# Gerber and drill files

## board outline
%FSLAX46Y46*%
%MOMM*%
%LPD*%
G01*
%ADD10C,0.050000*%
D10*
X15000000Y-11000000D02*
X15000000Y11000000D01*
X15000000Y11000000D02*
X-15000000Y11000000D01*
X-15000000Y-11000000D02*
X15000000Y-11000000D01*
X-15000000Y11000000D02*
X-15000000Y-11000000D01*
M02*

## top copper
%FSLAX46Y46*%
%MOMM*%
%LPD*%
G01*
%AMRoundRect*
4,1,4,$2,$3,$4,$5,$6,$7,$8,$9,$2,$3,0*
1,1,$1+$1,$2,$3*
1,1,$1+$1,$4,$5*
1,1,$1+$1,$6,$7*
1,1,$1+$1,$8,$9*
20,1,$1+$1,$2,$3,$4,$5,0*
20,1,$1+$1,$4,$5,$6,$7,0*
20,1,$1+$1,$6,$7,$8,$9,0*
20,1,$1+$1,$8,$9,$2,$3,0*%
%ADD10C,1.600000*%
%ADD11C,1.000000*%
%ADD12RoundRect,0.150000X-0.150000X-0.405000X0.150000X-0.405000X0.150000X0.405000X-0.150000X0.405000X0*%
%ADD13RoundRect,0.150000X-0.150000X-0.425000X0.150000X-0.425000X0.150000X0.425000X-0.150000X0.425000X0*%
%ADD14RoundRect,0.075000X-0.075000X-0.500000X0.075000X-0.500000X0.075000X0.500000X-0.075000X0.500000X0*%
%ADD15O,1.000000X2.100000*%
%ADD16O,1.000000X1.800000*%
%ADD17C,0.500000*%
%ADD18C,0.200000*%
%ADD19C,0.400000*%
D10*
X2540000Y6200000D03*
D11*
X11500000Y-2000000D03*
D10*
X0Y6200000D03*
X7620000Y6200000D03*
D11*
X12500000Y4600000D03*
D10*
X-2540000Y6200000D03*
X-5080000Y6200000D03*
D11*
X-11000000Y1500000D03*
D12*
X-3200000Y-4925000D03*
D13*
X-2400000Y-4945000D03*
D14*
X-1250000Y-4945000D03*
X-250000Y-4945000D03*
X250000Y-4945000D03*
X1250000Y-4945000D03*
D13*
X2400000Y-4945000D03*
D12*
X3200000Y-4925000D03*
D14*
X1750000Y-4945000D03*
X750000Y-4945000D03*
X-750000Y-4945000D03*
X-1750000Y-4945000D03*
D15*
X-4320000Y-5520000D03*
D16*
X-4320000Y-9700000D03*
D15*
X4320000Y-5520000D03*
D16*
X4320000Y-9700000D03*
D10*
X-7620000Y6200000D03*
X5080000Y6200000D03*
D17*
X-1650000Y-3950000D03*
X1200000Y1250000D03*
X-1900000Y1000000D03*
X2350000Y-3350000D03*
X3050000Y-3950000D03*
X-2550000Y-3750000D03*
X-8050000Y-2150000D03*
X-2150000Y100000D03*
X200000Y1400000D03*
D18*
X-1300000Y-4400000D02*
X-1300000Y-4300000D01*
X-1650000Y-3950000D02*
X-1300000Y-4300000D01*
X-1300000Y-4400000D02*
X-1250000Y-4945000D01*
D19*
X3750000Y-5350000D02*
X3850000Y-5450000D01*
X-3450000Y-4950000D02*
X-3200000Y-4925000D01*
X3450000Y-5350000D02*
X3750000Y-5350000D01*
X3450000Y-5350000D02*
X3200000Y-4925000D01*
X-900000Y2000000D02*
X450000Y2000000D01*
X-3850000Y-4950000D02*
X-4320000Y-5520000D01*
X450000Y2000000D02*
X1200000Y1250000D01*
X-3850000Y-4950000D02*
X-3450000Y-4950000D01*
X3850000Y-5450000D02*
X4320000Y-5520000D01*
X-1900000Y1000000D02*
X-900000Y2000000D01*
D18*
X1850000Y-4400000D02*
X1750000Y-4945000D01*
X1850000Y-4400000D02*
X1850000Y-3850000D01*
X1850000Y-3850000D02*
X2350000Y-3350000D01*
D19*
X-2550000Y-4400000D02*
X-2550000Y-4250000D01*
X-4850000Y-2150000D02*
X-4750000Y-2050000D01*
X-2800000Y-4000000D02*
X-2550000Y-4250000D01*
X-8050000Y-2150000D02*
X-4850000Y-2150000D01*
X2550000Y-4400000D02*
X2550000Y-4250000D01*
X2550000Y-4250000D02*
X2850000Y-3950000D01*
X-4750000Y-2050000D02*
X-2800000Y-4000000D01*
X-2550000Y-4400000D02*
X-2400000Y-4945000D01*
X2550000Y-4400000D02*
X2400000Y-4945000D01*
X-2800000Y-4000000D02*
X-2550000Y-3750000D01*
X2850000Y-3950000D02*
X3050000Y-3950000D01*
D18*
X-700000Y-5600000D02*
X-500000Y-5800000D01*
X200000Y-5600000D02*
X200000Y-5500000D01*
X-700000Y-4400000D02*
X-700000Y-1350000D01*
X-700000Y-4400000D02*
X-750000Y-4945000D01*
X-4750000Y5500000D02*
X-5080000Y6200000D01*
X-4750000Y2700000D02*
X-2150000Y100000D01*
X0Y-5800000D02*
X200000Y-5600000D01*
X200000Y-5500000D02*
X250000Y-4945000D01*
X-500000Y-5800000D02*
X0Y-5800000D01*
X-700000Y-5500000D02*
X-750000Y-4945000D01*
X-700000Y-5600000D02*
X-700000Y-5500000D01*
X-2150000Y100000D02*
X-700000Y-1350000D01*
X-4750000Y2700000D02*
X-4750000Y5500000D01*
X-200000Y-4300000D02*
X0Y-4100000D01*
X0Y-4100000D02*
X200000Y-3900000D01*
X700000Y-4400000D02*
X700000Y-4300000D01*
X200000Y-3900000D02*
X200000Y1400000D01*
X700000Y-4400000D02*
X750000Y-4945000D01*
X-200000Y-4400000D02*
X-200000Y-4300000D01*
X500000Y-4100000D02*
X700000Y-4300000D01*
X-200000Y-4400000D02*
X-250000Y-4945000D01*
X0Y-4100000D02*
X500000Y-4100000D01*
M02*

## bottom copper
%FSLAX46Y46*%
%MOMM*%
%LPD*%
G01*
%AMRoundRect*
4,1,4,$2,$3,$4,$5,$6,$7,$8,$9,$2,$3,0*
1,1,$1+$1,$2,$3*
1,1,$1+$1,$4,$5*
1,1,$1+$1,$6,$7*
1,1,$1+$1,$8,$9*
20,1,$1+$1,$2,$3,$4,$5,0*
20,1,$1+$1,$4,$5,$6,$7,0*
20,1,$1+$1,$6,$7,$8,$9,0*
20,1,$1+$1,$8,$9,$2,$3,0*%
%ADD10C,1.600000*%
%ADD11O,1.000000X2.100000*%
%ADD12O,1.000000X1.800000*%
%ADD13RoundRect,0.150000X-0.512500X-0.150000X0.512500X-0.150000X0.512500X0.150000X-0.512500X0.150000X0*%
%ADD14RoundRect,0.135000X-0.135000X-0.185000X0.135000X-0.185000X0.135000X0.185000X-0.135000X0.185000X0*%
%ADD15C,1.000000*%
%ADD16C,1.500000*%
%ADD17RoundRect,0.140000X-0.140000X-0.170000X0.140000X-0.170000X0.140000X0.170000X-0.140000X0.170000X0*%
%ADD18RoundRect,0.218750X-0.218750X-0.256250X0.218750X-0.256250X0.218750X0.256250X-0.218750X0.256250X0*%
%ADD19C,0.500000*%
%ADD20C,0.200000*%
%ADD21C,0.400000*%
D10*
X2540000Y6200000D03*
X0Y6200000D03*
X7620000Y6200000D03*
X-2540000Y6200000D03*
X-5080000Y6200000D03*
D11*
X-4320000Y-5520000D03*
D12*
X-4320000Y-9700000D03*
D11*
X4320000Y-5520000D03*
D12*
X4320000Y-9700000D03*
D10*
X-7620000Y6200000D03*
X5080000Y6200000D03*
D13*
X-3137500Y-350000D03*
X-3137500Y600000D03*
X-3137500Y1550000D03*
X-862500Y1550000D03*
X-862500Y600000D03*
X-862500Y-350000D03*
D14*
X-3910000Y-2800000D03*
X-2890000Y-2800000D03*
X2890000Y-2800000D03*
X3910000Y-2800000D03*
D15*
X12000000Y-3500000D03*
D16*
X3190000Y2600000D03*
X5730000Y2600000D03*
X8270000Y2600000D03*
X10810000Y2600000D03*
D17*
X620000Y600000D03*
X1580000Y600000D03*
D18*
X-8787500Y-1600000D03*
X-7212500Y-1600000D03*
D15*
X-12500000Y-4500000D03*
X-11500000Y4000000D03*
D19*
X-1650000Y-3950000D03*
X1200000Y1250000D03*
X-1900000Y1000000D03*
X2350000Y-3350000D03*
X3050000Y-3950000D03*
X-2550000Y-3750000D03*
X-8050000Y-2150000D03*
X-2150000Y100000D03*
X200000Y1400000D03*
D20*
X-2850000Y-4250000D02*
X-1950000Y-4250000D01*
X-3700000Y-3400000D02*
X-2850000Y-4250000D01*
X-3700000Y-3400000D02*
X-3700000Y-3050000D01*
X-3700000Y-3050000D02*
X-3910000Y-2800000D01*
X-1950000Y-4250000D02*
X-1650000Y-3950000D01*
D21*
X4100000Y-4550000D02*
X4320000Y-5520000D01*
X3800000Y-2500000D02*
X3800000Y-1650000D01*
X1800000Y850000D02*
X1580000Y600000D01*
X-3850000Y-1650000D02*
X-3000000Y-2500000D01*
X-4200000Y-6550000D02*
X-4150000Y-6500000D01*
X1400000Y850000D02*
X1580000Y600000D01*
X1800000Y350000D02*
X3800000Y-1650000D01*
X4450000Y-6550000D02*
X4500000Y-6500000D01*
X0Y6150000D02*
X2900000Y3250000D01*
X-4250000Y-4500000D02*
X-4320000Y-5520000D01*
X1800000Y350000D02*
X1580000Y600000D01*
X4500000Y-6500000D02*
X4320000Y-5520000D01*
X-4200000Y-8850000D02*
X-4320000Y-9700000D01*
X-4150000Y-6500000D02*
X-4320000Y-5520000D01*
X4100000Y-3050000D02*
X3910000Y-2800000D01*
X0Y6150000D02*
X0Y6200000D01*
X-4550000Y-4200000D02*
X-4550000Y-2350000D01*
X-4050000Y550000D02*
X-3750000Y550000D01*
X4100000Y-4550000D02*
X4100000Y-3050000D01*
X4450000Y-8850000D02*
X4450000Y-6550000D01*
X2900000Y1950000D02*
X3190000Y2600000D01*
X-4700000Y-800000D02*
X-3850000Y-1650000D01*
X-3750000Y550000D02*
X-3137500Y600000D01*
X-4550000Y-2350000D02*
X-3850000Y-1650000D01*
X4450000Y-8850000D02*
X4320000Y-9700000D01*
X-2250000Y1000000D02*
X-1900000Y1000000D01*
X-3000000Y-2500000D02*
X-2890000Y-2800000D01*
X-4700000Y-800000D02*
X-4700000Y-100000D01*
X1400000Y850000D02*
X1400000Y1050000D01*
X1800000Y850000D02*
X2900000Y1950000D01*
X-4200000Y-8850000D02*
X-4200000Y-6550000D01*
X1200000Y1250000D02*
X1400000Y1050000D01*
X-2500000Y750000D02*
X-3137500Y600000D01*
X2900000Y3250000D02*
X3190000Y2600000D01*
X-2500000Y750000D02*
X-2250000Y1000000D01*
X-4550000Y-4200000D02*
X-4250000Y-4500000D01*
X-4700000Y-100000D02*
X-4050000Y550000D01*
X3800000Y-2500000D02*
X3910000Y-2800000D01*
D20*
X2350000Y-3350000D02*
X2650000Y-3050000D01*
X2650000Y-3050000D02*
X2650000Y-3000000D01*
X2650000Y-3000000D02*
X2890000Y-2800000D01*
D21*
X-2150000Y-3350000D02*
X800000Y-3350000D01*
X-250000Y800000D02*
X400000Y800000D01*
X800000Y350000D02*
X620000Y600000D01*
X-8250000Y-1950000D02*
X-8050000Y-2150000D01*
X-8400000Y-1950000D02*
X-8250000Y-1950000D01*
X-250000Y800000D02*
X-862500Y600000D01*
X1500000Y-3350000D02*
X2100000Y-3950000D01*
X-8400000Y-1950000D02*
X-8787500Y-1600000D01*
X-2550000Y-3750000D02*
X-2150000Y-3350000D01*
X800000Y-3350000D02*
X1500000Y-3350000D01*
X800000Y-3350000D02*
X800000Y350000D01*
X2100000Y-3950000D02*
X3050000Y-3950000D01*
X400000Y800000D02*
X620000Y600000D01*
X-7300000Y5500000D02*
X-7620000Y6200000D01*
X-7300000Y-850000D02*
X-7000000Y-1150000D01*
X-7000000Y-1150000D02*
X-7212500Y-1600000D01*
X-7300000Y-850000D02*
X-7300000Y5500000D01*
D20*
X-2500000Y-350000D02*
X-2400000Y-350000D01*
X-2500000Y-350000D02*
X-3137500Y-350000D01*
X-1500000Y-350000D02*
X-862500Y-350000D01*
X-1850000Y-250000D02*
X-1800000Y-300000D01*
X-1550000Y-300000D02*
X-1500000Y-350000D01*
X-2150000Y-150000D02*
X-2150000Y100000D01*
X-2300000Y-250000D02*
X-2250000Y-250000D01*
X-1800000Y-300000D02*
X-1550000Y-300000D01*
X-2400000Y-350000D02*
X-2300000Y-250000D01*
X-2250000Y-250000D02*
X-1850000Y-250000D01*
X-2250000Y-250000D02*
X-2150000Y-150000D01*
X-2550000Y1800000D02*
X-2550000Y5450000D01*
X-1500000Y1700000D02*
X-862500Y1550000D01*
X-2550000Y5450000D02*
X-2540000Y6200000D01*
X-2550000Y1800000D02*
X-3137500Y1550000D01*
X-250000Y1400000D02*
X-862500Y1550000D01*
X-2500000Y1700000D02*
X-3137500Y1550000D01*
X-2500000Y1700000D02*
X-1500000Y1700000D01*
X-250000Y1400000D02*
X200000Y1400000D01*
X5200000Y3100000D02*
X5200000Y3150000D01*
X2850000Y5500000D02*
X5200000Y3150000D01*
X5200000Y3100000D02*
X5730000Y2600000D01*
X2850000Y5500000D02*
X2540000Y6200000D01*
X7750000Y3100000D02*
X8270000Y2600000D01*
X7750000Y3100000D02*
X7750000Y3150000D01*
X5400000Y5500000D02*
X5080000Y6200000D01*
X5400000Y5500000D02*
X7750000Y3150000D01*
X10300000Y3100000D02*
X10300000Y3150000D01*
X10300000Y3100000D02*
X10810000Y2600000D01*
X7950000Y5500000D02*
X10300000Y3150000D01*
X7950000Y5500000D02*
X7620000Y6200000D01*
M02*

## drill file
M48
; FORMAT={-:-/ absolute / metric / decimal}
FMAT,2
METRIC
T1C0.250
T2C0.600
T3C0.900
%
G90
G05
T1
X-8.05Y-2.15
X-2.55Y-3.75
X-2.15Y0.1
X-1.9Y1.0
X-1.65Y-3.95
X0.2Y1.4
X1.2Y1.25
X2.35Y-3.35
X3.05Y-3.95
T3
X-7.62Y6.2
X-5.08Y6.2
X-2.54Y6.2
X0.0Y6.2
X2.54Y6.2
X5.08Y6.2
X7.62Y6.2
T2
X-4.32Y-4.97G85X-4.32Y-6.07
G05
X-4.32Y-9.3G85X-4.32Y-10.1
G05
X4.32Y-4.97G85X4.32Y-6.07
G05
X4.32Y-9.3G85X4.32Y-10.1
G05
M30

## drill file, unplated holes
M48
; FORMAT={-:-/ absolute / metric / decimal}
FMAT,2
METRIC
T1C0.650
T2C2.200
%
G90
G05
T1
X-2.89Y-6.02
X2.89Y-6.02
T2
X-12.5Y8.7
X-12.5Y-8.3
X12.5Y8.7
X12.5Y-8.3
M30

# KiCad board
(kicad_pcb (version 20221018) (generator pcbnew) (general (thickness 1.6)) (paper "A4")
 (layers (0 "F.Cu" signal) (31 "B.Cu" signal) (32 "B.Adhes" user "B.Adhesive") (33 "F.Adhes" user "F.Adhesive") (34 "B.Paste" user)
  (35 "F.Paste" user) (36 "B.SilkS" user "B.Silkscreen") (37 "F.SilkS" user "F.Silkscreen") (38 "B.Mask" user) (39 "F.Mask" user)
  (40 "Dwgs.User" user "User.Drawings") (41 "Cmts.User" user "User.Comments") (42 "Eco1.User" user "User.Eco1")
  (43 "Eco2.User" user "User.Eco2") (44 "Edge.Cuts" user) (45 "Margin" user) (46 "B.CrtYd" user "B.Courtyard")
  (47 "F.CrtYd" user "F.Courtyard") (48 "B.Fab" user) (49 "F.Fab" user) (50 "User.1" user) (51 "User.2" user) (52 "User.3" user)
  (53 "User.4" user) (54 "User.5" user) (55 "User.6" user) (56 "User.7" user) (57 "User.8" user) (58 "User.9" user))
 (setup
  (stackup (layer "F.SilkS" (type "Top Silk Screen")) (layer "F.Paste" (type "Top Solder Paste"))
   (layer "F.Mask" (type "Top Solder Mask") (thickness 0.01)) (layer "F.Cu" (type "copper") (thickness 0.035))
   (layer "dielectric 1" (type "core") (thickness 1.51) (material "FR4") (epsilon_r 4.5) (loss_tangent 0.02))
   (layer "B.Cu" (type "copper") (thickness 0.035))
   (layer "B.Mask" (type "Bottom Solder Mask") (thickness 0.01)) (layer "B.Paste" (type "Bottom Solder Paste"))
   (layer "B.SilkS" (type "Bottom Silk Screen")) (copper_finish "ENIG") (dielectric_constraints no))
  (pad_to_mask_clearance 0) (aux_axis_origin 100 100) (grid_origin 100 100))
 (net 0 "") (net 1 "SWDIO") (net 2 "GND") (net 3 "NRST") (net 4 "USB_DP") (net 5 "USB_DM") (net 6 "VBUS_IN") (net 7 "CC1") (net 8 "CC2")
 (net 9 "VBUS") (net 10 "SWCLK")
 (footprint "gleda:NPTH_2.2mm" (layer "F.Cu") (at 112.5 91.3)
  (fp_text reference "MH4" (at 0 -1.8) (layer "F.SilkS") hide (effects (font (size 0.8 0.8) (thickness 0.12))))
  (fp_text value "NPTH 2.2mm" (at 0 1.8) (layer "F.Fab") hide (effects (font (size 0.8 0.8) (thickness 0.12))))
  (pad "" np_thru_hole circle (at 0 0) (size 2.2 2.2) (drill 2.2) (layers "*.Cu" "*.Mask")))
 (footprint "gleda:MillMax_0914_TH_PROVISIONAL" (layer "F.Cu") (at 102.54 93.8)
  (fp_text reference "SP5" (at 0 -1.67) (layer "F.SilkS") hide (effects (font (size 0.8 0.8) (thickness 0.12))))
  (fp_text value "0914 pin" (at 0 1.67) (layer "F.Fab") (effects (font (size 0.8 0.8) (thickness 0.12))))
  (pad "1" thru_hole circle (at 0 0) (size 1.6 1.6) (drill 0.9) (layers "*.Cu" "*.Mask") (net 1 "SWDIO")))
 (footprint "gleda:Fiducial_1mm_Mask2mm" (layer "F.Cu") (at 111.5 102)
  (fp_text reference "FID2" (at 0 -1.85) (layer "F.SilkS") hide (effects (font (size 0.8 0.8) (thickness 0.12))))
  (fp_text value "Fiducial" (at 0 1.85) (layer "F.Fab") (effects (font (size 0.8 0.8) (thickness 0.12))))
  (pad "" connect circle (at 0 0) (size 1 1) (layers "F.Cu" "F.Mask") (solder_mask_margin 0.5) (clearance 0.5)))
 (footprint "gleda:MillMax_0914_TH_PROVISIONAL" (layer "F.Cu") (at 100 93.8)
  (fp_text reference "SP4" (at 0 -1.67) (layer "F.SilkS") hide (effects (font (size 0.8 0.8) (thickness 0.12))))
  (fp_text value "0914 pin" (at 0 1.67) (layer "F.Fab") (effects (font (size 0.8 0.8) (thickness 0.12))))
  (pad "1" thru_hole circle (at 0 0) (size 1.6 1.6) (drill 0.9) (layers "*.Cu" "*.Mask") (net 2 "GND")))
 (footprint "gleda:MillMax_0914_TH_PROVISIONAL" (layer "F.Cu") (at 107.62 93.8)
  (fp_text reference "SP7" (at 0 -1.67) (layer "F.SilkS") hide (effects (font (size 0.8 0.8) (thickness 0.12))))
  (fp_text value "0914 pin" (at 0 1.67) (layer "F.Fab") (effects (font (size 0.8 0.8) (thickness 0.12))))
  (pad "1" thru_hole circle (at 0 0) (size 1.6 1.6) (drill 0.9) (layers "*.Cu" "*.Mask") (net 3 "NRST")))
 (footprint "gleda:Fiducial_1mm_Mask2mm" (layer "F.Cu") (at 112.5 95.4)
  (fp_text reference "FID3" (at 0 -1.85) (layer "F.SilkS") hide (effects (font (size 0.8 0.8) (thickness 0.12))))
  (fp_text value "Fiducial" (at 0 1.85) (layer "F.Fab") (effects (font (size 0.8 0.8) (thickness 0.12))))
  (pad "" connect circle (at 0 0) (size 1 1) (layers "F.Cu" "F.Mask") (solder_mask_margin 0.5) (clearance 0.5)))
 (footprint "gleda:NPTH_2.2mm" (layer "F.Cu") (at 87.5 91.3)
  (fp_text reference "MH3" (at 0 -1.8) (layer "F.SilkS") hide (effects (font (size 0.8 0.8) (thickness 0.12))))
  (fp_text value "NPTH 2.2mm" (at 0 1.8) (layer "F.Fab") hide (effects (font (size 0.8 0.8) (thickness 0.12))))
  (pad "" np_thru_hole circle (at 0 0) (size 2.2 2.2) (drill 2.2) (layers "*.Cu" "*.Mask")))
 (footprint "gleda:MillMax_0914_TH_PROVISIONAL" (layer "F.Cu") (at 97.46 93.8)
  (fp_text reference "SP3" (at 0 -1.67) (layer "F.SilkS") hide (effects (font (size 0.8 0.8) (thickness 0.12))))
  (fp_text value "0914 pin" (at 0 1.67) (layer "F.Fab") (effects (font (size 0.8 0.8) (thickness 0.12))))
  (pad "1" thru_hole circle (at 0 0) (size 1.6 1.6) (drill 0.9) (layers "*.Cu" "*.Mask") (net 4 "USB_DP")))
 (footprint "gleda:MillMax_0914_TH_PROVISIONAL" (layer "F.Cu") (at 94.92 93.8)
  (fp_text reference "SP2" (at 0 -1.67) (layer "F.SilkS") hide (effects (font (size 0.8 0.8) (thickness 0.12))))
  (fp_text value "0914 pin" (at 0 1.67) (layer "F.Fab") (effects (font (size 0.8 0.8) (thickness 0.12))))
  (pad "1" thru_hole circle (at 0 0) (size 1.6 1.6) (drill 0.9) (layers "*.Cu" "*.Mask") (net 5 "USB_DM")))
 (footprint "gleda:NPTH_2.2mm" (layer "F.Cu") (at 87.5 108.3)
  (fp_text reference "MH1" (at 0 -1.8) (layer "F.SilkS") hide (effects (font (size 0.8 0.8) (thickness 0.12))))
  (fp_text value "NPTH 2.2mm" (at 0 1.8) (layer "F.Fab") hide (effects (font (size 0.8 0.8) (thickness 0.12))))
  (pad "" np_thru_hole circle (at 0 0) (size 2.2 2.2) (drill 2.2) (layers "*.Cu" "*.Mask")))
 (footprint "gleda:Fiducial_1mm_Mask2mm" (layer "F.Cu") (at 89 98.5)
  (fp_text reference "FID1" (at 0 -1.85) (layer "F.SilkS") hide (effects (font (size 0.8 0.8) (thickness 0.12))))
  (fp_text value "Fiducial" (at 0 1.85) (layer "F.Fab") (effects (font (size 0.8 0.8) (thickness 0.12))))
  (pad "" connect circle (at 0 0) (size 1 1) (layers "F.Cu" "F.Mask") (solder_mask_margin 0.5) (clearance 0.5)))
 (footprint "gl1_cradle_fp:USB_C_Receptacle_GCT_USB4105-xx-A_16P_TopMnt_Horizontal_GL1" (layer "F.Cu") (at 100 108.625)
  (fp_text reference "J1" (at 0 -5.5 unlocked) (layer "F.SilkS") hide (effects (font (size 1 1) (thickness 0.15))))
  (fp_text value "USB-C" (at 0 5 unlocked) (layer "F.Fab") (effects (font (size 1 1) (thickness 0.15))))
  (pad "" np_thru_hole circle (at -2.89 -2.605) (size 0.65 0.65) (drill 0.65) (layers "F&B.Cu" "*.Mask"))
  (pad "" np_thru_hole circle (at 2.89 -2.605) (size 0.65 0.65) (drill 0.65) (layers "F&B.Cu" "*.Mask"))
  (pad "A1" smd roundrect (at -3.2 -3.7) (size 0.6 1.11) (layers "F.Cu" "F.Paste" "F.Mask") (roundrect_rratio 0.25) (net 2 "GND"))
  (pad "A4" smd roundrect (at -2.4 -3.68) (size 0.6 1.15) (layers "F.Cu" "F.Paste" "F.Mask") (roundrect_rratio 0.25) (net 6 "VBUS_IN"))
  (pad "A5" smd roundrect (at -1.25 -3.68) (size 0.3 1.15) (layers "F.Cu" "F.Paste" "F.Mask") (roundrect_rratio 0.25) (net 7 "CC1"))
  (pad "A6" smd roundrect (at -0.25 -3.68) (size 0.3 1.15) (layers "F.Cu" "F.Paste" "F.Mask") (roundrect_rratio 0.25) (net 4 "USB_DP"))
  (pad "A7" smd roundrect (at 0.25 -3.68) (size 0.3 1.15) (layers "F.Cu" "F.Paste" "F.Mask") (roundrect_rratio 0.25) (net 5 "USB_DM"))
  (pad "A8" smd roundrect (at 1.25 -3.68) (size 0.3 1.15) (layers "F.Cu" "F.Paste" "F.Mask") (roundrect_rratio 0.25))
  (pad "A9" smd roundrect (at 2.4 -3.68) (size 0.6 1.15) (layers "F.Cu" "F.Paste" "F.Mask") (roundrect_rratio 0.25) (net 6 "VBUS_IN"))
  (pad "A12" smd roundrect (at 3.2 -3.7) (size 0.6 1.11) (layers "F.Cu" "F.Paste" "F.Mask") (roundrect_rratio 0.25) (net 2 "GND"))
  (pad "B5" smd roundrect (at 1.75 -3.68) (size 0.3 1.15) (layers "F.Cu" "F.Paste" "F.Mask") (roundrect_rratio 0.25) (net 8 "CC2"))
  (pad "B6" smd roundrect (at 0.75 -3.68) (size 0.3 1.15) (layers "F.Cu" "F.Paste" "F.Mask") (roundrect_rratio 0.25) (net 4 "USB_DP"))
  (pad "B7" smd roundrect (at -0.75 -3.68) (size 0.3 1.15) (layers "F.Cu" "F.Paste" "F.Mask") (roundrect_rratio 0.25) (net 5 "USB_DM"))
  (pad "B8" smd roundrect (at -1.75 -3.68) (size 0.3 1.15) (layers "F.Cu" "F.Paste" "F.Mask") (roundrect_rratio 0.25))
  (pad "S1" thru_hole oval (at -4.32 -3.105) (size 1 2.1) (drill oval 0.6 1.7) (layers "*.Cu" "*.Mask" "F.Paste") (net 2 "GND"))
  (pad "S1" thru_hole oval (at -4.32 1.075) (size 1 1.8) (drill oval 0.6 1.4) (layers "*.Cu" "*.Mask" "F.Paste") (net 2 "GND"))
  (pad "S1" thru_hole oval (at 4.32 -3.105) (size 1 2.1) (drill oval 0.6 1.7) (layers "*.Cu" "*.Mask" "F.Paste") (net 2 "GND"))
  (pad "S1" thru_hole oval (at 4.32 1.075) (size 1 1.8) (drill oval 0.6 1.4) (layers "*.Cu" "*.Mask" "F.Paste") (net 2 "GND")))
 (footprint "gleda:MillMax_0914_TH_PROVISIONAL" (layer "F.Cu") (at 92.38 93.8)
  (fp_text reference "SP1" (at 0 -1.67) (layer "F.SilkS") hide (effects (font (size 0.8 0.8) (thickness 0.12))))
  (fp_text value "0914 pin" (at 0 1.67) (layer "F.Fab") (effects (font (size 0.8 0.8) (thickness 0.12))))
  (pad "1" thru_hole circle (at 0 0) (size 1.6 1.6) (drill 0.9) (layers "*.Cu" "*.Mask") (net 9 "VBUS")))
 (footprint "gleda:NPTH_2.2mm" (layer "F.Cu") (at 112.5 108.3)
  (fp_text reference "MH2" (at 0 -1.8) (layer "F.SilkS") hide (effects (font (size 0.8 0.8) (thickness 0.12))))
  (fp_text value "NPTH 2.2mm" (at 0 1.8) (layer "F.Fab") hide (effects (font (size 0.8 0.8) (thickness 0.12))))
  (pad "" np_thru_hole circle (at 0 0) (size 2.2 2.2) (drill 2.2) (layers "*.Cu" "*.Mask")))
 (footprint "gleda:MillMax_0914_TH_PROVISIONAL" (layer "F.Cu") (at 105.08 93.8)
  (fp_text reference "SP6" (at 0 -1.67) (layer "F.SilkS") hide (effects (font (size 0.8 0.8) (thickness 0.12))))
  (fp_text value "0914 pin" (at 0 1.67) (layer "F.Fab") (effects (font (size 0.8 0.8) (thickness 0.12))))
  (pad "1" thru_hole circle (at 0 0) (size 1.6 1.6) (drill 0.9) (layers "*.Cu" "*.Mask") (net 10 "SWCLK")))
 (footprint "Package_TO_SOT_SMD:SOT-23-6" (layer "B.Cu") (at 98 99.4)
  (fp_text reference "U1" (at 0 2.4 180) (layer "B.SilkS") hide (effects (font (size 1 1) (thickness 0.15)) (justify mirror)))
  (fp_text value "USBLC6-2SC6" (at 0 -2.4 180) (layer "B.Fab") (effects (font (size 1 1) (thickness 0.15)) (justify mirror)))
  (pad "1" smd roundrect (at -1.1375 0.95) (size 1.325 0.6) (layers "B.Cu" "B.Paste" "B.Mask") (roundrect_rratio 0.25) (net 5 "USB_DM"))
  (pad "2" smd roundrect (at -1.1375 0) (size 1.325 0.6) (layers "B.Cu" "B.Paste" "B.Mask") (roundrect_rratio 0.25) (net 2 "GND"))
  (pad "3" smd roundrect (at -1.1375 -0.95) (size 1.325 0.6) (layers "B.Cu" "B.Paste" "B.Mask") (roundrect_rratio 0.25) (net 4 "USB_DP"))
  (pad "4" smd roundrect (at 1.1375 -0.95) (size 1.325 0.6) (layers "B.Cu" "B.Paste" "B.Mask") (roundrect_rratio 0.25) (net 4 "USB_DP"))
  (pad "5" smd roundrect (at 1.1375 0) (size 1.325 0.6) (layers "B.Cu" "B.Paste" "B.Mask") (roundrect_rratio 0.25) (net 6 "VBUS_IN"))
  (pad "6" smd roundrect (at 1.1375 0.95) (size 1.325 0.6) (layers "B.Cu" "B.Paste" "B.Mask") (roundrect_rratio 0.25) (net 5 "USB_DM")))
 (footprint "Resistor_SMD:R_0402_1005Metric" (layer "B.Cu") (at 96.6 102.8)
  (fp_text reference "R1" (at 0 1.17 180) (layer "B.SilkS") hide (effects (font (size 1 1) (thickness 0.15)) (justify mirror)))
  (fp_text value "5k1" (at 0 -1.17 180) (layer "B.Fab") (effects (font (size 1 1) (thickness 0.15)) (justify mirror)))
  (pad "1" smd roundrect (at -0.51 0) (size 0.54 0.64) (layers "B.Cu" "B.Paste" "B.Mask") (roundrect_rratio 0.25) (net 7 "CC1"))
  (pad "2" smd roundrect (at 0.51 0) (size 0.54 0.64) (layers "B.Cu" "B.Paste" "B.Mask") (roundrect_rratio 0.25) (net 2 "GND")))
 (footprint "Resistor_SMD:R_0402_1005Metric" (layer "B.Cu") (at 103.4 102.8)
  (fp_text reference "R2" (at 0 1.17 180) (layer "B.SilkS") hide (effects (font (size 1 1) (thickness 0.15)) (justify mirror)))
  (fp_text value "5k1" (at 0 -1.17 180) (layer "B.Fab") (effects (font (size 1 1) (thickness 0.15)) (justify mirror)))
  (pad "1" smd roundrect (at -0.51 0) (size 0.54 0.64) (layers "B.Cu" "B.Paste" "B.Mask") (roundrect_rratio 0.25) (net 8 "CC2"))
  (pad "2" smd roundrect (at 0.51 0) (size 0.54 0.64) (layers "B.Cu" "B.Paste" "B.Mask") (roundrect_rratio 0.25) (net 2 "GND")))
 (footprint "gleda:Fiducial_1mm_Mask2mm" (layer "B.Cu") (at 112 103.5)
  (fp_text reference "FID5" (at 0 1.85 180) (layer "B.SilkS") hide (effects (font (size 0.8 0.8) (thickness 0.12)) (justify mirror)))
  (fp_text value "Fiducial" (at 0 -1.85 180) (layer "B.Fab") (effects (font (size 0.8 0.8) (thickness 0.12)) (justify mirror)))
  (pad "" connect circle (at 0 0) (size 1 1) (layers "B.Cu" "B.Mask") (solder_mask_margin 0.5) (clearance 0.5)))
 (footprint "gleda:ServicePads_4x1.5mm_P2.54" (layer "B.Cu") (at 107 97.4)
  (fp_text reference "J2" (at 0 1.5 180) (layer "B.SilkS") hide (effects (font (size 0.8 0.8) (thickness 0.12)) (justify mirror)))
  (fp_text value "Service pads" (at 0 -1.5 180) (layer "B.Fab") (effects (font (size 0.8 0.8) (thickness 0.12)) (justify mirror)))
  (pad "1" connect circle (at -3.81 0) (size 1.5 1.5) (layers "B.Cu" "B.Mask") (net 2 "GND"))
  (pad "2" connect circle (at -1.27 0) (size 1.5 1.5) (layers "B.Cu" "B.Mask") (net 1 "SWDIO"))
  (pad "3" connect circle (at 1.27 0) (size 1.5 1.5) (layers "B.Cu" "B.Mask") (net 10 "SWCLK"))
  (pad "4" connect circle (at 3.81 0) (size 1.5 1.5) (layers "B.Cu" "B.Mask") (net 3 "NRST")))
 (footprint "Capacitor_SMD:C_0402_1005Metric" (layer "B.Cu") (at 101.1 99.4)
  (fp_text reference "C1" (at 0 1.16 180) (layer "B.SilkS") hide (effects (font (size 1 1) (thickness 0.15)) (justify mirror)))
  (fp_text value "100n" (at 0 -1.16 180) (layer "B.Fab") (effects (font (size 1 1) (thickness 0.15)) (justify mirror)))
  (pad "1" smd roundrect (at -0.48 0) (size 0.56 0.62) (layers "B.Cu" "B.Paste" "B.Mask") (roundrect_rratio 0.25) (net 6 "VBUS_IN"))
  (pad "2" smd roundrect (at 0.48 0) (size 0.56 0.62) (layers "B.Cu" "B.Paste" "B.Mask") (roundrect_rratio 0.25) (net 2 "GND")))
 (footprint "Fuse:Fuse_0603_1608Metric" (layer "B.Cu") (at 92 101.6)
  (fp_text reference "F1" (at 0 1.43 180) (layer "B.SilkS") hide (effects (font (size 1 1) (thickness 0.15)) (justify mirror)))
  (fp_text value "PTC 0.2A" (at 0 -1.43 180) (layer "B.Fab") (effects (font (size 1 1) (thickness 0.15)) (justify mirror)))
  (pad "1" smd roundrect (at -0.7875 0) (size 0.875 0.95) (layers "B.Cu" "B.Paste" "B.Mask") (roundrect_rratio 0.25) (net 6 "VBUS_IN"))
  (pad "2" smd roundrect (at 0.7875 0) (size 0.875 0.95) (layers "B.Cu" "B.Paste" "B.Mask") (roundrect_rratio 0.25) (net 9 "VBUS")))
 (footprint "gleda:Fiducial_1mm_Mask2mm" (layer "B.Cu") (at 87.5 104.5)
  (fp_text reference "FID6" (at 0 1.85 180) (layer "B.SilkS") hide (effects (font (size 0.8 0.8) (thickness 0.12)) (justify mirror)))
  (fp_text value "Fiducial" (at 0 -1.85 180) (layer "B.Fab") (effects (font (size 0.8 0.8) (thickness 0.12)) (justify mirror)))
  (pad "" connect circle (at 0 0) (size 1 1) (layers "B.Cu" "B.Mask") (solder_mask_margin 0.5) (clearance 0.5)))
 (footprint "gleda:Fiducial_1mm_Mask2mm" (layer "B.Cu") (at 88.5 96)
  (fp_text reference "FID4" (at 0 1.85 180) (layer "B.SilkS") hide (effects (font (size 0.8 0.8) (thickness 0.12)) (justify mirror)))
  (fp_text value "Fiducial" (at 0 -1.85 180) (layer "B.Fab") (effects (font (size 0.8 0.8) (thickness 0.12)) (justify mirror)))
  (pad "" connect circle (at 0 0) (size 1 1) (layers "B.Cu" "B.Mask") (solder_mask_margin 0.5) (clearance 0.5)))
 (gr_line (start 115 111) (end 115 89) (stroke (width 0.05) (type default)) (layer "Edge.Cuts"))
 (gr_line (start 115 89) (end 85 89) (stroke (width 0.05) (type default)) (layer "Edge.Cuts"))
 (gr_line (start 85 111) (end 115 111) (stroke (width 0.05) (type default)) (layer "Edge.Cuts"))
 (gr_line (start 85 89) (end 85 111) (stroke (width 0.05) (type default)) (layer "Edge.Cuts"))
 (segment (start 98.7 104.4) (end 98.7 104.3) (width 0.2) (layer "F.Cu") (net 7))
 (segment (start 98.35 103.95) (end 98.7 104.3) (width 0.2) (layer "F.Cu") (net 7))
 (segment (start 98.7 104.4) (end 98.75 104.945) (width 0.2) (layer "F.Cu") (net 7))
 (via (at 98.35 103.95) (size 0.5) (drill 0.25) (layers "F.Cu" "B.Cu") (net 7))
 (segment (start 97.15 104.25) (end 98.05 104.25) (width 0.2) (layer "B.Cu") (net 7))
 (segment (start 96.3 103.4) (end 97.15 104.25) (width 0.2) (layer "B.Cu") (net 7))
 (segment (start 96.3 103.4) (end 96.3 103.05) (width 0.2) (layer "B.Cu") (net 7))
 (segment (start 96.3 103.05) (end 96.09 102.8) (width 0.2) (layer "B.Cu") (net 7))
 (segment (start 98.05 104.25) (end 98.35 103.95) (width 0.2) (layer "B.Cu") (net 7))
 (segment (start 103.75 105.35) (end 103.85 105.45) (width 0.4) (layer "F.Cu") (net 2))
 (segment (start 96.55 104.95) (end 96.8 104.925) (width 0.4) (layer "F.Cu") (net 2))
 (segment (start 103.45 105.35) (end 103.75 105.35) (width 0.4) (layer "F.Cu") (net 2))
 (segment (start 103.45 105.35) (end 103.2 104.925) (width 0.4) (layer "F.Cu") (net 2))
 (segment (start 99.1 98) (end 100.45 98) (width 0.4) (layer "F.Cu") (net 2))
 (segment (start 96.15 104.95) (end 95.68 105.52) (width 0.4) (layer "F.Cu") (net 2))
 (segment (start 100.45 98) (end 101.2 98.75) (width 0.4) (layer "F.Cu") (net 2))
 (segment (start 96.15 104.95) (end 96.55 104.95) (width 0.4) (layer "F.Cu") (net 2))
 (segment (start 103.85 105.45) (end 104.32 105.52) (width 0.4) (layer "F.Cu") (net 2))
 (segment (start 98.1 99) (end 99.1 98) (width 0.4) (layer "F.Cu") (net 2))
 (via (at 101.2 98.75) (size 0.5) (drill 0.25) (layers "F.Cu" "B.Cu") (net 2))
 (via (at 98.1 99) (size 0.5) (drill 0.25) (layers "F.Cu" "B.Cu") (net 2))
 (segment (start 104.1 104.55) (end 104.32 105.52) (width 0.4) (layer "B.Cu") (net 2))
 (segment (start 103.8 102.5) (end 103.8 101.65) (width 0.4) (layer "B.Cu") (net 2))
 (segment (start 101.8 99.15) (end 101.58 99.4) (width 0.4) (layer "B.Cu") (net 2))
 (segment (start 96.15 101.65) (end 97 102.5) (width 0.4) (layer "B.Cu") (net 2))
 (segment (start 95.8 106.55) (end 95.85 106.5) (width 0.4) (layer "B.Cu") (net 2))
 (segment (start 101.4 99.15) (end 101.58 99.4) (width 0.4) (layer "B.Cu") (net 2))
 (segment (start 101.8 99.65) (end 103.8 101.65) (width 0.4) (layer "B.Cu") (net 2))
 (segment (start 104.45 106.55) (end 104.5 106.5) (width 0.4) (layer "B.Cu") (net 2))
 (segment (start 100 93.85) (end 102.9 96.75) (width 0.4) (layer "B.Cu") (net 2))
 (segment (start 95.75 104.5) (end 95.68 105.52) (width 0.4) (layer "B.Cu") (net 2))
 (segment (start 101.8 99.65) (end 101.58 99.4) (width 0.4) (layer "B.Cu") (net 2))
 (segment (start 104.5 106.5) (end 104.32 105.52) (width 0.4) (layer "B.Cu") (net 2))
 (segment (start 95.8 108.85) (end 95.68 109.7) (width 0.4) (layer "B.Cu") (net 2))
 (segment (start 95.85 106.5) (end 95.68 105.52) (width 0.4) (layer "B.Cu") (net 2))
 (segment (start 104.1 103.05) (end 103.91 102.8) (width 0.4) (layer "B.Cu") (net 2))
 (segment (start 100 93.85) (end 100 93.8) (width 0.4) (layer "B.Cu") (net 2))
 (segment (start 95.45 104.2) (end 95.45 102.35) (width 0.4) (layer "B.Cu") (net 2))
 (segment (start 95.95 99.45) (end 96.25 99.45) (width 0.4) (layer "B.Cu") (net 2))
 (segment (start 104.1 104.55) (end 104.1 103.05) (width 0.4) (layer "B.Cu") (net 2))
 (segment (start 104.45 108.85) (end 104.45 106.55) (width 0.4) (layer "B.Cu") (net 2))
 (segment (start 102.9 98.05) (end 103.19 97.4) (width 0.4) (layer "B.Cu") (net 2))
 (segment (start 95.3 100.8) (end 96.15 101.65) (width 0.4) (layer "B.Cu") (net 2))
 (segment (start 96.25 99.45) (end 96.8625 99.4) (width 0.4) (layer "B.Cu") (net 2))
 (segment (start 95.45 102.35) (end 96.15 101.65) (width 0.4) (layer "B.Cu") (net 2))
 (segment (start 104.45 108.85) (end 104.32 109.7) (width 0.4) (layer "B.Cu") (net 2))
 (segment (start 97.75 99) (end 98.1 99) (width 0.4) (layer "B.Cu") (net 2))
 (segment (start 97 102.5) (end 97.11 102.8) (width 0.4) (layer "B.Cu") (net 2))
 (segment (start 95.3 100.8) (end 95.3 100.1) (width 0.4) (layer "B.Cu") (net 2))
 (segment (start 101.4 99.15) (end 101.4 98.95) (width 0.4) (layer "B.Cu") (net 2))
 (segment (start 101.8 99.15) (end 102.9 98.05) (width 0.4) (layer "B.Cu") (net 2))
 (segment (start 95.8 108.85) (end 95.8 106.55) (width 0.4) (layer "B.Cu") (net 2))
 (segment (start 101.2 98.75) (end 101.4 98.95) (width 0.4) (layer "B.Cu") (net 2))
 (segment (start 97.5 99.25) (end 96.8625 99.4) (width 0.4) (layer "B.Cu") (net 2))
 (segment (start 102.9 96.75) (end 103.19 97.4) (width 0.4) (layer "B.Cu") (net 2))
 (segment (start 97.5 99.25) (end 97.75 99) (width 0.4) (layer "B.Cu") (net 2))
 (segment (start 95.45 104.2) (end 95.75 104.5) (width 0.4) (layer "B.Cu") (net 2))
 (segment (start 95.3 100.1) (end 95.95 99.45) (width 0.4) (layer "B.Cu") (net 2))
 (segment (start 103.8 102.5) (end 103.91 102.8) (width 0.4) (layer "B.Cu") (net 2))
 (segment (start 101.85 104.4) (end 101.75 104.945) (width 0.2) (layer "F.Cu") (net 8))
 (segment (start 101.85 104.4) (end 101.85 103.85) (width 0.2) (layer "F.Cu") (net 8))
 (segment (start 101.85 103.85) (end 102.35 103.35) (width 0.2) (layer "F.Cu") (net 8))
 (via (at 102.35 103.35) (size 0.5) (drill 0.25) (layers "F.Cu" "B.Cu") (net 8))
 (segment (start 102.35 103.35) (end 102.65 103.05) (width 0.2) (layer "B.Cu") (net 8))
 (segment (start 102.65 103.05) (end 102.65 103) (width 0.2) (layer "B.Cu") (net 8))
 (segment (start 102.65 103) (end 102.89 102.8) (width 0.2) (layer "B.Cu") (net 8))
 (segment (start 97.45 104.4) (end 97.45 104.25) (width 0.4) (layer "F.Cu") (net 6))
 (segment (start 95.15 102.15) (end 95.25 102.05) (width 0.4) (layer "F.Cu") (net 6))
 (segment (start 97.2 104) (end 97.45 104.25) (width 0.4) (layer "F.Cu") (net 6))
 (segment (start 91.95 102.15) (end 95.15 102.15) (width 0.4) (layer "F.Cu") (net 6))
 (segment (start 102.55 104.4) (end 102.55 104.25) (width 0.4) (layer "F.Cu") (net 6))
 (segment (start 102.55 104.25) (end 102.85 103.95) (width 0.4) (layer "F.Cu") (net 6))
 (segment (start 95.25 102.05) (end 97.2 104) (width 0.4) (layer "F.Cu") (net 6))
 (segment (start 97.45 104.4) (end 97.6 104.945) (width 0.4) (layer "F.Cu") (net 6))
 (segment (start 102.55 104.4) (end 102.4 104.945) (width 0.4) (layer "F.Cu") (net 6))
 (segment (start 97.2 104) (end 97.45 103.75) (width 0.4) (layer "F.Cu") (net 6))
 (segment (start 102.85 103.95) (end 103.05 103.95) (width 0.4) (layer "F.Cu") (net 6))
 (via (at 103.05 103.95) (size 0.5) (drill 0.25) (layers "F.Cu" "B.Cu") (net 6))
 (via (at 97.45 103.75) (size 0.5) (drill 0.25) (layers "F.Cu" "B.Cu") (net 6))
 (via (at 91.95 102.15) (size 0.5) (drill 0.25) (layers "F.Cu" "B.Cu") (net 6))
 (segment (start 97.85 103.35) (end 100.8 103.35) (width 0.4) (layer "B.Cu") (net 6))
 (segment (start 99.75 99.2) (end 100.4 99.2) (width 0.4) (layer "B.Cu") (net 6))
 (segment (start 100.8 99.65) (end 100.62 99.4) (width 0.4) (layer "B.Cu") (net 6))
 (segment (start 91.75 101.95) (end 91.95 102.15) (width 0.4) (layer "B.Cu") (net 6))
 (segment (start 91.6 101.95) (end 91.75 101.95) (width 0.4) (layer "B.Cu") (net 6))
 (segment (start 99.75 99.2) (end 99.1375 99.4) (width 0.4) (layer "B.Cu") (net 6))
 (segment (start 101.5 103.35) (end 102.1 103.95) (width 0.4) (layer "B.Cu") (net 6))
 (segment (start 91.6 101.95) (end 91.2125 101.6) (width 0.4) (layer "B.Cu") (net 6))
 (segment (start 97.45 103.75) (end 97.85 103.35) (width 0.4) (layer "B.Cu") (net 6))
 (segment (start 100.8 103.35) (end 101.5 103.35) (width 0.4) (layer "B.Cu") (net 6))
 (segment (start 100.8 103.35) (end 100.8 99.65) (width 0.4) (layer "B.Cu") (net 6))
 (segment (start 102.1 103.95) (end 103.05 103.95) (width 0.4) (layer "B.Cu") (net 6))
 (segment (start 100.4 99.2) (end 100.62 99.4) (width 0.4) (layer "B.Cu") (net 6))
 (segment (start 92.7 94.5) (end 92.38 93.8) (width 0.4) (layer "B.Cu") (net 9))
 (segment (start 92.7 100.85) (end 93 101.15) (width 0.4) (layer "B.Cu") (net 9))
 (segment (start 93 101.15) (end 92.7875 101.6) (width 0.4) (layer "B.Cu") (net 9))
 (segment (start 92.7 100.85) (end 92.7 94.5) (width 0.4) (layer "B.Cu") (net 9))
 (segment (start 99.3 105.6) (end 99.5 105.8) (width 0.2) (layer "F.Cu") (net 5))
 (segment (start 100.2 105.6) (end 100.2 105.5) (width 0.2) (layer "F.Cu") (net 5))
 (segment (start 99.3 104.4) (end 99.3 101.35) (width 0.2) (layer "F.Cu") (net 5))
 (segment (start 99.3 104.4) (end 99.25 104.945) (width 0.2) (layer "F.Cu") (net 5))
 (segment (start 95.25 94.5) (end 94.92 93.8) (width 0.2) (layer "F.Cu") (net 5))
 (segment (start 95.25 97.3) (end 97.85 99.9) (width 0.2) (layer "F.Cu") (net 5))
 (segment (start 100 105.8) (end 100.2 105.6) (width 0.2) (layer "F.Cu") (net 5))
 (segment (start 100.2 105.5) (end 100.25 104.945) (width 0.2) (layer "F.Cu") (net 5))
 (segment (start 99.5 105.8) (end 100 105.8) (width 0.2) (layer "F.Cu") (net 5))
 (segment (start 99.3 105.5) (end 99.25 104.945) (width 0.2) (layer "F.Cu") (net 5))
 (segment (start 99.3 105.6) (end 99.3 105.5) (width 0.2) (layer "F.Cu") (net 5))
 (segment (start 97.85 99.9) (end 99.3 101.35) (width 0.2) (layer "F.Cu") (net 5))
 (segment (start 95.25 97.3) (end 95.25 94.5) (width 0.2) (layer "F.Cu") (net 5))
 (via (at 97.85 99.9) (size 0.5) (drill 0.25) (layers "F.Cu" "B.Cu") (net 5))
 (segment (start 97.5 100.35) (end 97.6 100.35) (width 0.2) (layer "B.Cu") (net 5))
 (segment (start 97.5 100.35) (end 96.8625 100.35) (width 0.2) (layer "B.Cu") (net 5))
 (segment (start 98.5 100.35) (end 99.1375 100.35) (width 0.2) (layer "B.Cu") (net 5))
 (segment (start 98.15 100.25) (end 98.2 100.3) (width 0.2) (layer "B.Cu") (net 5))
 (segment (start 98.45 100.3) (end 98.5 100.35) (width 0.2) (layer "B.Cu") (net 5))
 (segment (start 97.85 100.15) (end 97.85 99.9) (width 0.2) (layer "B.Cu") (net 5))
 (segment (start 97.7 100.25) (end 97.75 100.25) (width 0.2) (layer "B.Cu") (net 5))
 (segment (start 98.2 100.3) (end 98.45 100.3) (width 0.2) (layer "B.Cu") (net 5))
 (segment (start 97.6 100.35) (end 97.7 100.25) (width 0.2) (layer "B.Cu") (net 5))
 (segment (start 97.75 100.25) (end 98.15 100.25) (width 0.2) (layer "B.Cu") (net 5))
 (segment (start 97.75 100.25) (end 97.85 100.15) (width 0.2) (layer "B.Cu") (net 5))
 (segment (start 99.8 104.3) (end 100 104.1) (width 0.2) (layer "F.Cu") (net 4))
 (segment (start 100 104.1) (end 100.2 103.9) (width 0.2) (layer "F.Cu") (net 4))
 (segment (start 100.7 104.4) (end 100.7 104.3) (width 0.2) (layer "F.Cu") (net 4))
 (segment (start 100.2 103.9) (end 100.2 98.6) (width 0.2) (layer "F.Cu") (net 4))
 (segment (start 100.7 104.4) (end 100.75 104.945) (width 0.2) (layer "F.Cu") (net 4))
 (segment (start 99.8 104.4) (end 99.8 104.3) (width 0.2) (layer "F.Cu") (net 4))
 (segment (start 100.5 104.1) (end 100.7 104.3) (width 0.2) (layer "F.Cu") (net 4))
 (segment (start 99.8 104.4) (end 99.75 104.945) (width 0.2) (layer "F.Cu") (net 4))
 (segment (start 100 104.1) (end 100.5 104.1) (width 0.2) (layer "F.Cu") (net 4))
 (via (at 100.2 98.6) (size 0.5) (drill 0.25) (layers "F.Cu" "B.Cu") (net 4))
 (segment (start 97.45 98.2) (end 97.45 94.55) (width 0.2) (layer "B.Cu") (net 4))
 (segment (start 98.5 98.3) (end 99.1375 98.45) (width 0.2) (layer "B.Cu") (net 4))
 (segment (start 97.45 94.55) (end 97.46 93.8) (width 0.2) (layer "B.Cu") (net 4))
 (segment (start 97.45 98.2) (end 96.8625 98.45) (width 0.2) (layer "B.Cu") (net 4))
 (segment (start 99.75 98.6) (end 99.1375 98.45) (width 0.2) (layer "B.Cu") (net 4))
 (segment (start 97.5 98.3) (end 96.8625 98.45) (width 0.2) (layer "B.Cu") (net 4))
 (segment (start 97.5 98.3) (end 98.5 98.3) (width 0.2) (layer "B.Cu") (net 4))
 (segment (start 99.75 98.6) (end 100.2 98.6) (width 0.2) (layer "B.Cu") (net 4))
 (segment (start 105.2 96.9) (end 105.2 96.85) (width 0.2) (layer "B.Cu") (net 1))
 (segment (start 102.85 94.5) (end 105.2 96.85) (width 0.2) (layer "B.Cu") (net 1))
 (segment (start 105.2 96.9) (end 105.73 97.4) (width 0.2) (layer "B.Cu") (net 1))
 (segment (start 102.85 94.5) (end 102.54 93.8) (width 0.2) (layer "B.Cu") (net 1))
 (segment (start 107.75 96.9) (end 108.27 97.4) (width 0.2) (layer "B.Cu") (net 10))
 (segment (start 107.75 96.9) (end 107.75 96.85) (width 0.2) (layer "B.Cu") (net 10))
 (segment (start 105.4 94.5) (end 105.08 93.8) (width 0.2) (layer "B.Cu") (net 10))
 (segment (start 105.4 94.5) (end 107.75 96.85) (width 0.2) (layer "B.Cu") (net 10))
 (segment (start 110.3 96.9) (end 110.3 96.85) (width 0.2) (layer "B.Cu") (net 3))
 (segment (start 110.3 96.9) (end 110.81 97.4) (width 0.2) (layer "B.Cu") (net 3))
 (segment (start 107.95 94.5) (end 110.3 96.85) (width 0.2) (layer "B.Cu") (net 3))
 (segment (start 107.95 94.5) (end 107.62 93.8) (width 0.2) (layer "B.Cu") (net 3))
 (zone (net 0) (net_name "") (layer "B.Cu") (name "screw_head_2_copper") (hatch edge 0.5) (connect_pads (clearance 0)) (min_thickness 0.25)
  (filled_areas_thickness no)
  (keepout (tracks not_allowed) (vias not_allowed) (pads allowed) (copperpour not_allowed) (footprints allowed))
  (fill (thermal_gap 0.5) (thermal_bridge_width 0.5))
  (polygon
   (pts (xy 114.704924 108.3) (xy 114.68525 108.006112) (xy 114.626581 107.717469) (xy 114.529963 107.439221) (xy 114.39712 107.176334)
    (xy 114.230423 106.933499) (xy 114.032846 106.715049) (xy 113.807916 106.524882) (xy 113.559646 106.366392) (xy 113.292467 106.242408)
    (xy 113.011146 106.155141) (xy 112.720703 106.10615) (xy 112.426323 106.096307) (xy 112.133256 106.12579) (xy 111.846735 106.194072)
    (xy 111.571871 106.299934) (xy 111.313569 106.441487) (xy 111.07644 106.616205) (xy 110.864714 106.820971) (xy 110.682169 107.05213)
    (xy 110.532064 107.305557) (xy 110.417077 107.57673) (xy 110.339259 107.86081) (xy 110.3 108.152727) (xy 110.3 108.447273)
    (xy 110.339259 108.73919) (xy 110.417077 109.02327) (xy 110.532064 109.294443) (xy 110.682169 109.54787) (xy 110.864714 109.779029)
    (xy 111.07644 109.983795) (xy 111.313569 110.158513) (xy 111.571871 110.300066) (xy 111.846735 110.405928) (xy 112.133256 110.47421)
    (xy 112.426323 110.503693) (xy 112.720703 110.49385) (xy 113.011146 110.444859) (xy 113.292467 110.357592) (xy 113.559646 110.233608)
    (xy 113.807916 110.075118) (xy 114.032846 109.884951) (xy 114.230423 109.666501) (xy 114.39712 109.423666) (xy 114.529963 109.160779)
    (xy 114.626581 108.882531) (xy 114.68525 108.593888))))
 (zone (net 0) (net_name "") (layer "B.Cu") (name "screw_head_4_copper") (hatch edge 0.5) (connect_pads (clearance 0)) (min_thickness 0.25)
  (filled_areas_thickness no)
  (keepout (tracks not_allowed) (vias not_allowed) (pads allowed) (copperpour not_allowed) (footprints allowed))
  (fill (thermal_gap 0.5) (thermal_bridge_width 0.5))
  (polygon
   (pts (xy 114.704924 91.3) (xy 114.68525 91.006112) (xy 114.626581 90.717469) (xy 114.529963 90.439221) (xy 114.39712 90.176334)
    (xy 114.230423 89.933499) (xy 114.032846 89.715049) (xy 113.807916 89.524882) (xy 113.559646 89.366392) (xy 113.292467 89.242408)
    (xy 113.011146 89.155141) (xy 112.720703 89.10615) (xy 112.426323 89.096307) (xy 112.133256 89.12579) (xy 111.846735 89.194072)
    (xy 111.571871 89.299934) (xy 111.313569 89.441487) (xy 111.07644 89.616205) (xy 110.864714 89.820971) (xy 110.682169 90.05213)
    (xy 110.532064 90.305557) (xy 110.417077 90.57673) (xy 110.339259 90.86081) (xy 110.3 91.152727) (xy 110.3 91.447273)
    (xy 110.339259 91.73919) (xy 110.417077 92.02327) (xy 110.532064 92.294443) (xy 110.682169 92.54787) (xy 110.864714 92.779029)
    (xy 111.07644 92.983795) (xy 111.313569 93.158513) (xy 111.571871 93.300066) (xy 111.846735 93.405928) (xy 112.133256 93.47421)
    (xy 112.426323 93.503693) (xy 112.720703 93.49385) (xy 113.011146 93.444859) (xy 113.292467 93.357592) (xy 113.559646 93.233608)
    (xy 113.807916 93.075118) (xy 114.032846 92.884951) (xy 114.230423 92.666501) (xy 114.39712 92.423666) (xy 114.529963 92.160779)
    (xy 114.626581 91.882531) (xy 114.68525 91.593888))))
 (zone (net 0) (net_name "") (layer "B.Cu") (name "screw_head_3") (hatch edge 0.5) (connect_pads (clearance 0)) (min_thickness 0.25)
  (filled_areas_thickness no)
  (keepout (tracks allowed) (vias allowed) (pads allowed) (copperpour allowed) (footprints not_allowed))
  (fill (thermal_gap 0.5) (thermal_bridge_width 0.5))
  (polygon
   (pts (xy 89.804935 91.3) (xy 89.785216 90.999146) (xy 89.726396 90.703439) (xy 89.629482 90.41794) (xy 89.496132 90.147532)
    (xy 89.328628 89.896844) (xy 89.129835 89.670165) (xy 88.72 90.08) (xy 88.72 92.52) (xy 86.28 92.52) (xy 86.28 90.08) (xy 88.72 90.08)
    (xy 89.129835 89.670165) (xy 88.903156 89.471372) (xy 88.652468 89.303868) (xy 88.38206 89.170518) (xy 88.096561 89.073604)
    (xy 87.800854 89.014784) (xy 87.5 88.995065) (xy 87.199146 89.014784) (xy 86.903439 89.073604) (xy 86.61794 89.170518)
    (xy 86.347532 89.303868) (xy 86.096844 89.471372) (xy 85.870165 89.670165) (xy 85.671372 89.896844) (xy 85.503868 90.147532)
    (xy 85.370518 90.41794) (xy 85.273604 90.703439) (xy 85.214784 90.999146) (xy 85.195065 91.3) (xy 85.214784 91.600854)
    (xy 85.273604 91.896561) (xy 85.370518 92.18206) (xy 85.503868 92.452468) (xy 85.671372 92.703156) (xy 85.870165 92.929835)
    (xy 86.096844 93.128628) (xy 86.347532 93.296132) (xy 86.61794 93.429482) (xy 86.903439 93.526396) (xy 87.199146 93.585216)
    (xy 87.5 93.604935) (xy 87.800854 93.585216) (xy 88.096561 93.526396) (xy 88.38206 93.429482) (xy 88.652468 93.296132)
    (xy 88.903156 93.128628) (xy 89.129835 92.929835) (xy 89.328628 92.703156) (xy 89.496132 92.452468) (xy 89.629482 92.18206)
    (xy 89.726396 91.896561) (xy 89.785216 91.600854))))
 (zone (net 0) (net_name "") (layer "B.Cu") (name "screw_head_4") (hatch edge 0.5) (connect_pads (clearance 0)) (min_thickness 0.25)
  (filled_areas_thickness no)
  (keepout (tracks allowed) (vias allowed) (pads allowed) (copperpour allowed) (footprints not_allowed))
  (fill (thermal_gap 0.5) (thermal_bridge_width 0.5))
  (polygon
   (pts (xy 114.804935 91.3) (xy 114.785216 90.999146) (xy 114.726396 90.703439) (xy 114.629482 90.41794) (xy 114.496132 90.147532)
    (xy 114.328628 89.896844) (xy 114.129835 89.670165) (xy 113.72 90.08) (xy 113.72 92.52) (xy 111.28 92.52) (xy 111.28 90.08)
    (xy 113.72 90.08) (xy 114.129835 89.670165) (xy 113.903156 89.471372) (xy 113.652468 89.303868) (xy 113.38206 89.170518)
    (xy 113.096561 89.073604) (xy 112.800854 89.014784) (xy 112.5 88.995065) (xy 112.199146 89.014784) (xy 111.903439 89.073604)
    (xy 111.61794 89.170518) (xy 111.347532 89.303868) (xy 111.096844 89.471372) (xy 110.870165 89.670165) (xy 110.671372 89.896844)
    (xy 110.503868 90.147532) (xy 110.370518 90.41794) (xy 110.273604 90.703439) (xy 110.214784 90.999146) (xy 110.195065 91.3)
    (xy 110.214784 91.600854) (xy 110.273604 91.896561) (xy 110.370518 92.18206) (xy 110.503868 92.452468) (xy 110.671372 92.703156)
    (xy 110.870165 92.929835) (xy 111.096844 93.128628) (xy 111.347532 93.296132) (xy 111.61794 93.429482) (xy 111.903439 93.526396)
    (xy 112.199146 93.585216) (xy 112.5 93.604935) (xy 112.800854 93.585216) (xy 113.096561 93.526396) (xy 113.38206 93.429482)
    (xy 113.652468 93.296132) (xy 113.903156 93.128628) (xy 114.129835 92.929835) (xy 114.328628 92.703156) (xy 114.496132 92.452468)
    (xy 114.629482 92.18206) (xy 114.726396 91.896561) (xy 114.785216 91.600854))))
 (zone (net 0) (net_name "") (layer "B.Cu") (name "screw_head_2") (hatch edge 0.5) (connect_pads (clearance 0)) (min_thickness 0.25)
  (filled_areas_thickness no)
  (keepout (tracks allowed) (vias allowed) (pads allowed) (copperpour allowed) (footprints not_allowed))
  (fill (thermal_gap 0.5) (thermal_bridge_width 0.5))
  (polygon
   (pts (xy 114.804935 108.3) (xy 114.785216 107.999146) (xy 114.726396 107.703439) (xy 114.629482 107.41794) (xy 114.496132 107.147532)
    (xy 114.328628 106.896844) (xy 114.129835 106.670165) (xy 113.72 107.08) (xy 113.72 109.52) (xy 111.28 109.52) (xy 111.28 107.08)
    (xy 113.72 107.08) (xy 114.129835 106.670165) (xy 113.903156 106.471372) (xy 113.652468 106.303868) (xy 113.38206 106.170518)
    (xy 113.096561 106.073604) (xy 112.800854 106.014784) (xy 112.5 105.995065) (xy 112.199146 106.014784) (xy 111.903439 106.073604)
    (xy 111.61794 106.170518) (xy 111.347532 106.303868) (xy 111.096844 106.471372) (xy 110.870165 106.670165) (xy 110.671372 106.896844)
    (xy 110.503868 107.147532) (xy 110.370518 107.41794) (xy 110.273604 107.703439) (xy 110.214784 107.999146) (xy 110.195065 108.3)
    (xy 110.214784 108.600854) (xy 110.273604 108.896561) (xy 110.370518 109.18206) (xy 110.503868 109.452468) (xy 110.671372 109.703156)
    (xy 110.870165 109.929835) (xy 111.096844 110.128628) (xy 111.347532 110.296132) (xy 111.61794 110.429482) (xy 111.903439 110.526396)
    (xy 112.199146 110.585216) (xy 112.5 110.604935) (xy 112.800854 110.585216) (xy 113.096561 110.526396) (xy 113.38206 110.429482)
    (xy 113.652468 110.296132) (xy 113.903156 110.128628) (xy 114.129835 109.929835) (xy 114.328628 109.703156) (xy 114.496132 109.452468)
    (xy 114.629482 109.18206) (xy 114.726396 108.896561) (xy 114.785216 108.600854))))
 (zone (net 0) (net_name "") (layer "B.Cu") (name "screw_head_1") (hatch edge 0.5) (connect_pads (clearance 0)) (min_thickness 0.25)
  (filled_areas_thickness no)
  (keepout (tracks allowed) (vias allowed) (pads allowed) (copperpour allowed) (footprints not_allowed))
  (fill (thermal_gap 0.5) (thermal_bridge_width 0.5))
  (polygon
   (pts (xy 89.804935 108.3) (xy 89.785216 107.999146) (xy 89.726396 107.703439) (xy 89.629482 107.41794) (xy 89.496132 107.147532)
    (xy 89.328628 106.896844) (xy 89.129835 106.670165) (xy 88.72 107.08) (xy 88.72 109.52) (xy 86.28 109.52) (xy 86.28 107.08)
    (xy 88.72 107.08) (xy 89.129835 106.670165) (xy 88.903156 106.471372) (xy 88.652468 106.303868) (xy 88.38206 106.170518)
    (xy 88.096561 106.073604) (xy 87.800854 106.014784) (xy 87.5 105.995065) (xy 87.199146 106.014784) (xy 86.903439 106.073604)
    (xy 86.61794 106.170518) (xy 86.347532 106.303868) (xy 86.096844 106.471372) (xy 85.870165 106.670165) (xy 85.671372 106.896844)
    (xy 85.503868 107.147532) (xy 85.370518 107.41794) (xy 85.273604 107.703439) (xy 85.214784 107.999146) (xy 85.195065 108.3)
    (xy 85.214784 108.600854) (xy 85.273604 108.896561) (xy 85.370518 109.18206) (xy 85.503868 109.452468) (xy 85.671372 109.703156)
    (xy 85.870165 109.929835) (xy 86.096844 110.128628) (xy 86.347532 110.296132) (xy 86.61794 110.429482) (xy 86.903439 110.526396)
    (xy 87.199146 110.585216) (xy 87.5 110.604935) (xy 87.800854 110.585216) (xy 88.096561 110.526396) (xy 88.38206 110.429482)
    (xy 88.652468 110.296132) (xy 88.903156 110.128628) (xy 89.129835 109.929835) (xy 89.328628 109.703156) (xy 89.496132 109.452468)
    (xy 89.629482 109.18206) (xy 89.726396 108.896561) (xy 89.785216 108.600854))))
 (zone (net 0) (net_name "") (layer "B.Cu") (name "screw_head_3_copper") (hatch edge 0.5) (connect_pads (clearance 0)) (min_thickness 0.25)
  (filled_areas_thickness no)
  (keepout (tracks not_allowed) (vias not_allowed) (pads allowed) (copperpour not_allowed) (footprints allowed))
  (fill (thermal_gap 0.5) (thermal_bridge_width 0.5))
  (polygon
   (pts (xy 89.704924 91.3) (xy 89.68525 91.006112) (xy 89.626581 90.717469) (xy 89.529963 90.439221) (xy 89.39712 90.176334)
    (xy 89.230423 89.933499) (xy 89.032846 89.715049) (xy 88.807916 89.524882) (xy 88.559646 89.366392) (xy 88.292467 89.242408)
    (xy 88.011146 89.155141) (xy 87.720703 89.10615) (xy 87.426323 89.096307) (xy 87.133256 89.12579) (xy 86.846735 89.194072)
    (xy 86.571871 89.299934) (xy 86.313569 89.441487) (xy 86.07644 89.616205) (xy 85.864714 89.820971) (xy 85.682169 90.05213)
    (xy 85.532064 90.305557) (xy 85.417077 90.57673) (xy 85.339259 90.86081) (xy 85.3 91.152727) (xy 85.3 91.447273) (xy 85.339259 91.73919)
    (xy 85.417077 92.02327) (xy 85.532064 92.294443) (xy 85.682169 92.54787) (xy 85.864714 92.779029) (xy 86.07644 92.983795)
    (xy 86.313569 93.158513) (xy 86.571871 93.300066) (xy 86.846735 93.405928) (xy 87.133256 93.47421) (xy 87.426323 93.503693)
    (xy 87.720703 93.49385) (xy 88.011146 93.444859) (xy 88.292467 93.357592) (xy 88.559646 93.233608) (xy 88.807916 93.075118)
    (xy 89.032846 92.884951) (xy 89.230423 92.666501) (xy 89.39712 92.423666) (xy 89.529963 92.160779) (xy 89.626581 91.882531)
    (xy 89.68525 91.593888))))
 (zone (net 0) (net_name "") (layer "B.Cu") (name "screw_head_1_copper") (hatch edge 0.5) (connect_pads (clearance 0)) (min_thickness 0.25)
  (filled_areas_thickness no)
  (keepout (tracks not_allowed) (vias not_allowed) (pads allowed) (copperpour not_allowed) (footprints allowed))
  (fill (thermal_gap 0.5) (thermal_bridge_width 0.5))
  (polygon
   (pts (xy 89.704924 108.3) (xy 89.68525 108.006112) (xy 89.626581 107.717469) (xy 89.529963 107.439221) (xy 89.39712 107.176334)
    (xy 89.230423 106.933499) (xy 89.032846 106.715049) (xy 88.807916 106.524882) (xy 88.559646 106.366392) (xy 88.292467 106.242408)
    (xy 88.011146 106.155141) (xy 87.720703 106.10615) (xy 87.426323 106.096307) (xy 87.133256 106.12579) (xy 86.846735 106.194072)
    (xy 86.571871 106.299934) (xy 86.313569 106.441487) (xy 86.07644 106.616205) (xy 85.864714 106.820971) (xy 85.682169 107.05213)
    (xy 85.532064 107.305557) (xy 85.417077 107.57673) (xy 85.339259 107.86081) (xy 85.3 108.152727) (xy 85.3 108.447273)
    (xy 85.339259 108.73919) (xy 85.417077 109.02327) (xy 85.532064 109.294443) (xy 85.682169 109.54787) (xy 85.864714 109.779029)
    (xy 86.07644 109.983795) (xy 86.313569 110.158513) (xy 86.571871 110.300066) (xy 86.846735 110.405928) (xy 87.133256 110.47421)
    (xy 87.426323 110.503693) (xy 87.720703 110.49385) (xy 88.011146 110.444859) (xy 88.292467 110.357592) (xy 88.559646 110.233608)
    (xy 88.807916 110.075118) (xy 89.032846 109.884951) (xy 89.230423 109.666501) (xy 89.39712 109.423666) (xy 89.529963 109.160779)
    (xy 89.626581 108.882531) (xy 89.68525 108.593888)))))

